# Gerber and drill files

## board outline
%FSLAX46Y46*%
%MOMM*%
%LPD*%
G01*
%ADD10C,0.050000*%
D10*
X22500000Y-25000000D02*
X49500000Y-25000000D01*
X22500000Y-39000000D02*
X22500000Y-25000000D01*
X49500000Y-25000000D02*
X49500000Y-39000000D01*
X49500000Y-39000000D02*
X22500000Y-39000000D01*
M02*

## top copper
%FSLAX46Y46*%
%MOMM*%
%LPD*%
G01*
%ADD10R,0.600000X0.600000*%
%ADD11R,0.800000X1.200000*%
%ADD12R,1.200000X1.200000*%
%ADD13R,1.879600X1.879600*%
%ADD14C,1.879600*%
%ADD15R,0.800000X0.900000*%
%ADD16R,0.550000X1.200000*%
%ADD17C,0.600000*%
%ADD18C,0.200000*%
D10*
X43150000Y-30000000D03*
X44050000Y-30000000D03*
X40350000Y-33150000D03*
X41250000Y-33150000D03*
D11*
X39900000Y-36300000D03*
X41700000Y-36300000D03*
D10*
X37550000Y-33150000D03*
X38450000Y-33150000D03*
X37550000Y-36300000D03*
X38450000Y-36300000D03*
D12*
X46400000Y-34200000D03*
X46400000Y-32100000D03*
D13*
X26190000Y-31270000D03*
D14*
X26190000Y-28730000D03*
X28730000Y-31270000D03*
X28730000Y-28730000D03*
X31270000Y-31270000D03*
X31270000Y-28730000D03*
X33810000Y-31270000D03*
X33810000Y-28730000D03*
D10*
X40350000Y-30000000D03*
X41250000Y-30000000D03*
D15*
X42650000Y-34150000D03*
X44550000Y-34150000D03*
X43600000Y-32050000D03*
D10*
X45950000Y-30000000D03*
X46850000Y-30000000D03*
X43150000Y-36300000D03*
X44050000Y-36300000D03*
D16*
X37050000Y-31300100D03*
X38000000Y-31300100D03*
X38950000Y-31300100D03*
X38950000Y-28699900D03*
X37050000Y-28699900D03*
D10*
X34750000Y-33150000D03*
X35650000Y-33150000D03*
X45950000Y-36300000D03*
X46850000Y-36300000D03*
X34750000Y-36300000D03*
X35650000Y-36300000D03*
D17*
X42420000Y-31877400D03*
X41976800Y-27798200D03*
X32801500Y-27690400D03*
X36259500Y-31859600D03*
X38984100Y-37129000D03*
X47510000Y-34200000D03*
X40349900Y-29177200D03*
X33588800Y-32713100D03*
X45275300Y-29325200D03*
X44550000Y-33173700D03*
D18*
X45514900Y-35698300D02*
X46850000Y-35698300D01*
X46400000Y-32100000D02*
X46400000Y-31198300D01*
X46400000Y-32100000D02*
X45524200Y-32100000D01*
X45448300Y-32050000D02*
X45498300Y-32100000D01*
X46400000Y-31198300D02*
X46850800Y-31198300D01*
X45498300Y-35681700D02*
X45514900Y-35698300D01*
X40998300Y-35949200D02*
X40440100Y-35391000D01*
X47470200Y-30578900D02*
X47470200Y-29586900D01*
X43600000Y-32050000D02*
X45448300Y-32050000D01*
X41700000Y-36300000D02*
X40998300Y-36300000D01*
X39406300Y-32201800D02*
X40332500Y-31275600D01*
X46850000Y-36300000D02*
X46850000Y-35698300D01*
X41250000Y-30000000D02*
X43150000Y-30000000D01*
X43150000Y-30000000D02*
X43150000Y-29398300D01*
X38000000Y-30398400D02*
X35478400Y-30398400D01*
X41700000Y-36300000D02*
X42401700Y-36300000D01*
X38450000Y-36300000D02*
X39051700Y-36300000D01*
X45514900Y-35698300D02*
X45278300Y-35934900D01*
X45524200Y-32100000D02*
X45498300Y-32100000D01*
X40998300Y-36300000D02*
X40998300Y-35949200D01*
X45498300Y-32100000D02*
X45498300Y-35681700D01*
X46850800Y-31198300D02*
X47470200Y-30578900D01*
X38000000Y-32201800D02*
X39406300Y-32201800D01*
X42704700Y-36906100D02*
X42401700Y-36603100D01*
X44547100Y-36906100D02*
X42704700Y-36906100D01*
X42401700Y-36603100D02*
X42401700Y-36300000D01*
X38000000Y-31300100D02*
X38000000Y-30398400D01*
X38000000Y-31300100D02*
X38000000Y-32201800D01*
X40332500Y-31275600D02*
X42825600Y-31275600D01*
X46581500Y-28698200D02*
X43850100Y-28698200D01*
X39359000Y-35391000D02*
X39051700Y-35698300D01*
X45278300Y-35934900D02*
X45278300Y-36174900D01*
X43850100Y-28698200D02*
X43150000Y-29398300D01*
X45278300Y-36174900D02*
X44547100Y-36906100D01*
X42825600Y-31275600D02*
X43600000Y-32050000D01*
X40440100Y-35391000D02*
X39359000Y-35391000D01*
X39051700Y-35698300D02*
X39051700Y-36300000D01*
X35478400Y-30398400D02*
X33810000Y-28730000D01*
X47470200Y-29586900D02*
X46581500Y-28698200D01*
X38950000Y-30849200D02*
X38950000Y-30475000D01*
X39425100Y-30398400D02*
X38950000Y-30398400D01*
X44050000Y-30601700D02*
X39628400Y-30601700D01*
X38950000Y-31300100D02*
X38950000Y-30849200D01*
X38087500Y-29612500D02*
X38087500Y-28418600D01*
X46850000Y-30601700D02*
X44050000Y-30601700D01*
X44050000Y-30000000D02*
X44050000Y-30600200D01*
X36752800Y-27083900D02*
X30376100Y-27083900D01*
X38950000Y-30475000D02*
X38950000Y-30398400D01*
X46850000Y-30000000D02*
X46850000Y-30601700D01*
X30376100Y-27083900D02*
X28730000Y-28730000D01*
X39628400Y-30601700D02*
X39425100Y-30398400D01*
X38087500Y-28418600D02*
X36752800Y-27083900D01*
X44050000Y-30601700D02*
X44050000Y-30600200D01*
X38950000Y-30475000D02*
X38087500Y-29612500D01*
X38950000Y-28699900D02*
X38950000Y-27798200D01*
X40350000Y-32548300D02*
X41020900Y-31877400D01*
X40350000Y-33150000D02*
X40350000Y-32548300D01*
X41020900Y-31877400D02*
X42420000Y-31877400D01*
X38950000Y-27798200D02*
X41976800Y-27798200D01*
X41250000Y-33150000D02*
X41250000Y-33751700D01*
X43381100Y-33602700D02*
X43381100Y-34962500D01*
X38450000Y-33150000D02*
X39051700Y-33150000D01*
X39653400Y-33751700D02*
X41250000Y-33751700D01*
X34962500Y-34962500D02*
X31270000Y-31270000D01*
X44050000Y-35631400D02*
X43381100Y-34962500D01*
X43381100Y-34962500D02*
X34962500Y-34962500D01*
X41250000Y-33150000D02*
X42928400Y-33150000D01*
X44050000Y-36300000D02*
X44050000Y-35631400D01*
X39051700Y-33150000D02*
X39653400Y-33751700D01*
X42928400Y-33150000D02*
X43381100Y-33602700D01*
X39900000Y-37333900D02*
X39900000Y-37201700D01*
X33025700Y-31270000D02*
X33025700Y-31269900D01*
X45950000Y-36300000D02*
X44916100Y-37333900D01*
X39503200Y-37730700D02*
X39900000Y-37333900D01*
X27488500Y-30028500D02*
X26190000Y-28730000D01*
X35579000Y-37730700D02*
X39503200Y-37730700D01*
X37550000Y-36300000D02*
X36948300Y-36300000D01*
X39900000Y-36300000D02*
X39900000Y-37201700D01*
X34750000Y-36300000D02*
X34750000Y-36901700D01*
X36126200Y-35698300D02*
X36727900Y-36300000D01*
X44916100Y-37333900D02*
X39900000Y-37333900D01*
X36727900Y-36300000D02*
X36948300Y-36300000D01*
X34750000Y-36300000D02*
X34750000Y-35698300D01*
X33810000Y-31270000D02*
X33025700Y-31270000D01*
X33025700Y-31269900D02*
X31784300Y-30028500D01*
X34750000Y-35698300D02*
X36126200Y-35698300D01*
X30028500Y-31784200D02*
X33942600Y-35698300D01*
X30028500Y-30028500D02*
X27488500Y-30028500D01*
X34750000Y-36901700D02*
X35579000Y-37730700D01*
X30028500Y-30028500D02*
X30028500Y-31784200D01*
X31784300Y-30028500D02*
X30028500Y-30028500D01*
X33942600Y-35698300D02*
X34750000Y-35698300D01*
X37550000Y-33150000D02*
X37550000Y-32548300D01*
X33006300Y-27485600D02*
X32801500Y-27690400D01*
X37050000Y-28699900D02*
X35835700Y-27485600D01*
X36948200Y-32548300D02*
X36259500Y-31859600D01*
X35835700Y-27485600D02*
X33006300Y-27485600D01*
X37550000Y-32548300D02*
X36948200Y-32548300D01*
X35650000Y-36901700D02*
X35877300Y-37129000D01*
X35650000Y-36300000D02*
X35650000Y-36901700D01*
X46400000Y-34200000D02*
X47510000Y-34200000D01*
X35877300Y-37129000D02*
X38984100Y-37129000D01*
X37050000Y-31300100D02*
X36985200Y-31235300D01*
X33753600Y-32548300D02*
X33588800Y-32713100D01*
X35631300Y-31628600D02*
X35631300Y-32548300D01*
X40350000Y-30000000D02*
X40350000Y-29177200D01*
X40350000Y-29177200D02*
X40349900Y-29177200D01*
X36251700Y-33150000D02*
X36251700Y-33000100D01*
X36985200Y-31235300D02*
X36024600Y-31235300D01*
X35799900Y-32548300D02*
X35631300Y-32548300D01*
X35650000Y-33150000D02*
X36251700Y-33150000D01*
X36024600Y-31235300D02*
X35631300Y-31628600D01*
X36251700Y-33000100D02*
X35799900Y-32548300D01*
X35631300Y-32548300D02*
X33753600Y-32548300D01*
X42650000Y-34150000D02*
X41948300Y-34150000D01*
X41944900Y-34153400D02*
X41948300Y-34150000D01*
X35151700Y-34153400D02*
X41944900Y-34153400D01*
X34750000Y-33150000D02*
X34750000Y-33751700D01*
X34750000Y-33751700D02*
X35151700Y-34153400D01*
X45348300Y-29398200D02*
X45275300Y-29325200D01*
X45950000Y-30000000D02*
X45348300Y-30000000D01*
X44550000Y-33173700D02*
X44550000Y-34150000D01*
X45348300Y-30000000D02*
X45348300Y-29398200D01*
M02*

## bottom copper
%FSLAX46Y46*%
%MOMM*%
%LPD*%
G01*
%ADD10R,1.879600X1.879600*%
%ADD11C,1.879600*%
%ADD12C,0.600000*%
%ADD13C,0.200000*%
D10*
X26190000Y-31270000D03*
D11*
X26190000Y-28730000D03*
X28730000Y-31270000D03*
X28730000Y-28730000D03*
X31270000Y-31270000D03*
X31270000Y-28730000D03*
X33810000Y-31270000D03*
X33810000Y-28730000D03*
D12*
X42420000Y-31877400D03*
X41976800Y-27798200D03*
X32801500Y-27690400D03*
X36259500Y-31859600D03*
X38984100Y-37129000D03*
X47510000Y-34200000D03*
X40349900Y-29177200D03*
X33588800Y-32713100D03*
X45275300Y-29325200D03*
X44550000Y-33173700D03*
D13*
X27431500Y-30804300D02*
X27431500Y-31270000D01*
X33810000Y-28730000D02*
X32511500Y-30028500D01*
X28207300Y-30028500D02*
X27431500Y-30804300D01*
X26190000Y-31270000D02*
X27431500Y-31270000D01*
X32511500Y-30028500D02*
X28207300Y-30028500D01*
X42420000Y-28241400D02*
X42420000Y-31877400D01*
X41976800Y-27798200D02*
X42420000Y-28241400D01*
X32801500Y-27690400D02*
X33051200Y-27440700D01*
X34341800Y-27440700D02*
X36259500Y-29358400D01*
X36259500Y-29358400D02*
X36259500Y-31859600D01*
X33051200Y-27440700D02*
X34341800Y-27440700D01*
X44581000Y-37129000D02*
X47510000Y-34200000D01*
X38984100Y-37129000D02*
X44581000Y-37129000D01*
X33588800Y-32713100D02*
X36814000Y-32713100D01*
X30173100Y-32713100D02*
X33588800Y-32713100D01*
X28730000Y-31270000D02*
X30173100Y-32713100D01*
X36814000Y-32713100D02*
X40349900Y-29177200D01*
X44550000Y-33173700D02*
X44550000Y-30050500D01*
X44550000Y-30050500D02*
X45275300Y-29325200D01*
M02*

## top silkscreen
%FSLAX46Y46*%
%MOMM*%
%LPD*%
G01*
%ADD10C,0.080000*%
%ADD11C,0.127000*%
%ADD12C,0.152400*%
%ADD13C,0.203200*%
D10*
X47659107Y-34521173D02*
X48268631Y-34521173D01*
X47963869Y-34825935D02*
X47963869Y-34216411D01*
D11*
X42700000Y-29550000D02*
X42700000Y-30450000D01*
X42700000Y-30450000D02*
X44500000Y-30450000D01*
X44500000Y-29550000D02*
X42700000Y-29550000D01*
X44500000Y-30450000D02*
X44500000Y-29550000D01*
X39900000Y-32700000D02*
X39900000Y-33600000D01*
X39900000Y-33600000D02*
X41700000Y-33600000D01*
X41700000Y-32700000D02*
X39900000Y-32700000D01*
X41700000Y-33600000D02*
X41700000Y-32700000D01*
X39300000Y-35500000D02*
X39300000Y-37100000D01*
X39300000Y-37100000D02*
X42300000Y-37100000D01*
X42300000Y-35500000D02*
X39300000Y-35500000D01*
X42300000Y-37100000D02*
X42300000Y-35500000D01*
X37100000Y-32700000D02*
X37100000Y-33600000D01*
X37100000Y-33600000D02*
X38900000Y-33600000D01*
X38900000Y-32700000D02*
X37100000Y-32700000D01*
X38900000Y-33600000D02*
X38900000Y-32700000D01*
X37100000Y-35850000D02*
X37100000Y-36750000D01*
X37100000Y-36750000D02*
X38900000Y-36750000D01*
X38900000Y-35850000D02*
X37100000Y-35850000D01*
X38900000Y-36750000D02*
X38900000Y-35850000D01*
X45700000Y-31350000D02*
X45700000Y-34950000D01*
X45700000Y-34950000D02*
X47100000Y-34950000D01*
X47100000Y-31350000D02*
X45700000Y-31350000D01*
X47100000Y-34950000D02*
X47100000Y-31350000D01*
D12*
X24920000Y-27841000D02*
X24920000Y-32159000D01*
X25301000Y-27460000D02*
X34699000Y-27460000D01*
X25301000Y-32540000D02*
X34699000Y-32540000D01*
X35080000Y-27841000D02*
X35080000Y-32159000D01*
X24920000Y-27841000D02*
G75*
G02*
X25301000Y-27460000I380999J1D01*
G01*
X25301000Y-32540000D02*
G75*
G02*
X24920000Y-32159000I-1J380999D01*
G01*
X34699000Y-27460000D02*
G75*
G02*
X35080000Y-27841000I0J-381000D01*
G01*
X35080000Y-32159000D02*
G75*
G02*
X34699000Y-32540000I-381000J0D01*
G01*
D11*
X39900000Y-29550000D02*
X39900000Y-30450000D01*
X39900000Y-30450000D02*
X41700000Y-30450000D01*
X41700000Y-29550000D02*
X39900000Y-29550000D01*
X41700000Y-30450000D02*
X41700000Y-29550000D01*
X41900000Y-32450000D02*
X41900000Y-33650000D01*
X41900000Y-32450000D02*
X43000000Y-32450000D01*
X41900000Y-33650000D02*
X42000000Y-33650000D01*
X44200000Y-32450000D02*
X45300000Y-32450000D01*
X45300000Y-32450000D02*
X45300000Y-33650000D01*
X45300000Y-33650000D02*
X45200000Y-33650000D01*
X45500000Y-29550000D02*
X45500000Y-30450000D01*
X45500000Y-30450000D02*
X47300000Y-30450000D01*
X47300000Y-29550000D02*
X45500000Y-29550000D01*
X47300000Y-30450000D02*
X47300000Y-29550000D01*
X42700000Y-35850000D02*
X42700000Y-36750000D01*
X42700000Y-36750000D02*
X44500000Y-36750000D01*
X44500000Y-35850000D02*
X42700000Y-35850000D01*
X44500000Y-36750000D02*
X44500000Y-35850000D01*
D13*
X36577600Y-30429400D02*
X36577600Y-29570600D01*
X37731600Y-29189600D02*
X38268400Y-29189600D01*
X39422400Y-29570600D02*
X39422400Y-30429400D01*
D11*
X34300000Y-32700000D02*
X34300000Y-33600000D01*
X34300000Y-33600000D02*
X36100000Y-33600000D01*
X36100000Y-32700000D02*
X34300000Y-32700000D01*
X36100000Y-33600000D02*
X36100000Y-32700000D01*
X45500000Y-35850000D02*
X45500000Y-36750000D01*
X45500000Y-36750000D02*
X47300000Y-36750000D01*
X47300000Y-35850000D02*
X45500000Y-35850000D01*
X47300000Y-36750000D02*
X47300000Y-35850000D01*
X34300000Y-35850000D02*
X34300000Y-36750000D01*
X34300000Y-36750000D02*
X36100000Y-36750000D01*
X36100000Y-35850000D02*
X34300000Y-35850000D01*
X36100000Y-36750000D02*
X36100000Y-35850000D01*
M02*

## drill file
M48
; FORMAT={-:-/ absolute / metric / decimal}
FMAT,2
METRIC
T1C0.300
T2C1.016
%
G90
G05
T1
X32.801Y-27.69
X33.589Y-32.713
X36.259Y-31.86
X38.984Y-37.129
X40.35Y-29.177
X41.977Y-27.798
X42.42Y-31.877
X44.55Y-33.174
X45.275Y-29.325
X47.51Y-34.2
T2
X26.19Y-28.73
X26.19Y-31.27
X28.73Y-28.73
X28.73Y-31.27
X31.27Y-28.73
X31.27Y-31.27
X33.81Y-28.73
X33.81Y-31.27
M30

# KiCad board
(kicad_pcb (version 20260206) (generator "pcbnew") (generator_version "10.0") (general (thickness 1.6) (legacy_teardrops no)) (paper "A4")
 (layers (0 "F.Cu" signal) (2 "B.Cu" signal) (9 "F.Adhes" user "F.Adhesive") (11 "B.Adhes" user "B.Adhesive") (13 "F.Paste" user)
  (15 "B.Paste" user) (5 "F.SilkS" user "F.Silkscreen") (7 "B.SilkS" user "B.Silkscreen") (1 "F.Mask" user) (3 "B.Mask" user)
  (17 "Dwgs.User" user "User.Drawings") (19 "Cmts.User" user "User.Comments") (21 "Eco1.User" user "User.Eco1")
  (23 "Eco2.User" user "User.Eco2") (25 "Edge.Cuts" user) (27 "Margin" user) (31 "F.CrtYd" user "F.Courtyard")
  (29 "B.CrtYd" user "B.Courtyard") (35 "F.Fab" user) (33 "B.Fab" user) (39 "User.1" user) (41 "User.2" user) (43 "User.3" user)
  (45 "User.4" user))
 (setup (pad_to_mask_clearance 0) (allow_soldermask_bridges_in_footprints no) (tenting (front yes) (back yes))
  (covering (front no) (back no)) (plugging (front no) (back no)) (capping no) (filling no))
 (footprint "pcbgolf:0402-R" (layer "F.Cu") (at 43.6 30)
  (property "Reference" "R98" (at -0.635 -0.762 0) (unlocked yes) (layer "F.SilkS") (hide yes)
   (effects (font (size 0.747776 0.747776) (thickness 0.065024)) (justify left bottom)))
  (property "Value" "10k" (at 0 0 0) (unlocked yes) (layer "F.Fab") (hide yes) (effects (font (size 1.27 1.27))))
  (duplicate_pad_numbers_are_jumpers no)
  (fp_line (start -0.9 -0.45) (end -0.9 0.45) (stroke (width 0.127) (type solid)) (layer "F.SilkS"))
  (fp_line (start -0.9 0.45) (end 0.9 0.45) (stroke (width 0.127) (type solid)) (layer "F.SilkS"))
  (fp_line (start 0.9 -0.45) (end -0.9 -0.45) (stroke (width 0.127) (type solid)) (layer "F.SilkS"))
  (fp_line (start 0.9 0.45) (end 0.9 -0.45) (stroke (width 0.127) (type solid)) (layer "F.SilkS"))
  (pad "1" smd rect (at -0.45 0) (size 0.6 0.6) (layers "F.Cu" "F.Mask" "F.Paste") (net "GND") (solder_mask_margin 0.0508)
   (solder_paste_margin 0) (thermal_bridge_angle 0))
  (pad "2" smd rect (at 0.45 0) (size 0.6 0.6) (layers "F.Cu" "F.Mask" "F.Paste") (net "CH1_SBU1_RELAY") (solder_mask_margin 0.0508)
   (solder_paste_margin 0) (thermal_bridge_angle 0)))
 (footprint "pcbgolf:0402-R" (layer "F.Cu") (at 40.8 33.15)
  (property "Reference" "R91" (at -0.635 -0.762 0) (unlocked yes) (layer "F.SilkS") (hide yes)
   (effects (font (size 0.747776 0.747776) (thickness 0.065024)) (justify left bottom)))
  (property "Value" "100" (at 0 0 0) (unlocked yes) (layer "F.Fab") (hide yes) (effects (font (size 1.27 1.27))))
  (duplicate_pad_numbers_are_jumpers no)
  (fp_line (start -0.9 -0.45) (end -0.9 0.45) (stroke (width 0.127) (type solid)) (layer "F.SilkS"))
  (fp_line (start -0.9 0.45) (end 0.9 0.45) (stroke (width 0.127) (type solid)) (layer "F.SilkS"))
  (fp_line (start 0.9 -0.45) (end -0.9 -0.45) (stroke (width 0.127) (type solid)) (layer "F.SilkS"))
  (fp_line (start 0.9 0.45) (end 0.9 -0.45) (stroke (width 0.127) (type solid)) (layer "F.SilkS"))
  (pad "1" smd rect (at -0.45 0) (size 0.6 0.6) (layers "F.Cu" "F.Mask" "F.Paste") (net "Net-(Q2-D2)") (solder_mask_margin 0.0508)
   (solder_paste_margin 0) (thermal_bridge_angle 0))
  (pad "2" smd rect (at 0.45 0) (size 0.6 0.6) (layers "F.Cu" "F.Mask" "F.Paste") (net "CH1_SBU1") (solder_mask_margin 0.0508)
   (solder_paste_margin 0) (thermal_bridge_angle 0)))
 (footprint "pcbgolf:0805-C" (layer "F.Cu") (at 40.8 36.3)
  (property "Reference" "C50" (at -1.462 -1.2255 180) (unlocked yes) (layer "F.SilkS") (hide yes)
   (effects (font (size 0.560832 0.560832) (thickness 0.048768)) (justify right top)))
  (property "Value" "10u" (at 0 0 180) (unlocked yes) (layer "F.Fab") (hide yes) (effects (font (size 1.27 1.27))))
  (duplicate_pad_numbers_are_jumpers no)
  (fp_line (start -1.5 -0.8) (end -1.5 0.8) (stroke (width 0.127) (type solid)) (layer "F.SilkS"))
  (fp_line (start -1.5 0.8) (end 1.5 0.8) (stroke (width 0.127) (type solid)) (layer "F.SilkS"))
  (fp_line (start 1.5 -0.8) (end -1.5 -0.8) (stroke (width 0.127) (type solid)) (layer "F.SilkS"))
  (fp_line (start 1.5 0.8) (end 1.5 -0.8) (stroke (width 0.127) (type solid)) (layer "F.SilkS"))
  (pad "1" smd rect (at -0.9 0) (size 0.8 1.2) (layers "F.Cu" "F.Mask" "F.Paste") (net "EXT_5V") (solder_mask_margin 0.0508)
   (solder_paste_margin 0) (thermal_bridge_angle 0))
  (pad "2" smd rect (at 0.9 0) (size 0.8 1.2) (layers "F.Cu" "F.Mask" "F.Paste") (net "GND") (solder_mask_margin 0.0508)
   (solder_paste_margin 0) (thermal_bridge_angle 0)))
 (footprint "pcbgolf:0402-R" (layer "F.Cu") (at 38 33.15)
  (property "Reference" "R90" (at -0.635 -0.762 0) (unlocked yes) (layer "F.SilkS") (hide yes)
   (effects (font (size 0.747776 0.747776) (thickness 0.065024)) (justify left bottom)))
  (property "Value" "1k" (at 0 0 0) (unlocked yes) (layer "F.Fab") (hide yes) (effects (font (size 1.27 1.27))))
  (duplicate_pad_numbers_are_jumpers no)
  (fp_line (start -0.9 -0.45) (end -0.9 0.45) (stroke (width 0.127) (type solid)) (layer "F.SilkS"))
  (fp_line (start -0.9 0.45) (end 0.9 0.45) (stroke (width 0.127) (type solid)) (layer "F.SilkS"))
  (fp_line (start 0.9 -0.45) (end -0.9 -0.45) (stroke (width 0.127) (type solid)) (layer "F.SilkS"))
  (fp_line (start 0.9 0.45) (end 0.9 -0.45) (stroke (width 0.127) (type solid)) (layer "F.SilkS"))
  (pad "1" smd rect (at -0.45 0) (size 0.6 0.6) (layers "F.Cu" "F.Mask" "F.Paste") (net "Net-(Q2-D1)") (solder_mask_margin 0.0508)
   (solder_paste_margin 0) (thermal_bridge_angle 0))
  (pad "2" smd rect (at 0.45 0) (size 0.6 0.6) (layers "F.Cu" "F.Mask" "F.Paste") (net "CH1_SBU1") (solder_mask_margin 0.0508)
   (solder_paste_margin 0) (thermal_bridge_angle 0)))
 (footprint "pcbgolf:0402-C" (layer "F.Cu") (at 38 36.3)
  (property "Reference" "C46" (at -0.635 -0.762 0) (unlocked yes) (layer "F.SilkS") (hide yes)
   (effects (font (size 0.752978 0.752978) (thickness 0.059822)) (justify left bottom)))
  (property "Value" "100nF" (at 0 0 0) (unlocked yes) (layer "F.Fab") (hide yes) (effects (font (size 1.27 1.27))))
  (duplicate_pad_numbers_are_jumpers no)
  (fp_line (start -0.9 -0.45) (end -0.9 0.45) (stroke (width 0.127) (type solid)) (layer "F.SilkS"))
  (fp_line (start -0.9 0.45) (end 0.9 0.45) (stroke (width 0.127) (type solid)) (layer "F.SilkS"))
  (fp_line (start 0.9 -0.45) (end -0.9 -0.45) (stroke (width 0.127) (type solid)) (layer "F.SilkS"))
  (fp_line (start 0.9 0.45) (end 0.9 -0.45) (stroke (width 0.127) (type solid)) (layer "F.SilkS"))
  (pad "1" smd rect (at -0.45 0) (size 0.6 0.6) (layers "F.Cu" "F.Mask" "F.Paste") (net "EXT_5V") (solder_mask_margin 0.0508)
   (solder_paste_margin 0) (thermal_bridge_angle 0))
  (pad "2" smd rect (at 0.45 0) (size 0.6 0.6) (layers "F.Cu" "F.Mask" "F.Paste") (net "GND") (solder_mask_margin 0.0508)
   (solder_paste_margin 0) (thermal_bridge_angle 0)))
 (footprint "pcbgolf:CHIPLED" (layer "F.Cu") (at 46.4 33.15)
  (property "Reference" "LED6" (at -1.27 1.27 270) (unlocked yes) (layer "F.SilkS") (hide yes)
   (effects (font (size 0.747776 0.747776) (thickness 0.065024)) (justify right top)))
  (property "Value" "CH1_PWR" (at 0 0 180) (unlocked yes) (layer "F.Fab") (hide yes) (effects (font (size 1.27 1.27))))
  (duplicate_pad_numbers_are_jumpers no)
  (fp_line (start -0.7 -1.8) (end -0.7 1.8) (stroke (width 0.127) (type solid)) (layer "F.SilkS"))
  (fp_line (start -0.7 1.8) (end 0.7 1.8) (stroke (width 0.127) (type solid)) (layer "F.SilkS"))
  (fp_line (start 0.7 -1.8) (end -0.7 -1.8) (stroke (width 0.127) (type solid)) (layer "F.SilkS"))
  (fp_line (start 0.7 1.8) (end 0.7 -1.8) (stroke (width 0.127) (type solid)) (layer "F.SilkS"))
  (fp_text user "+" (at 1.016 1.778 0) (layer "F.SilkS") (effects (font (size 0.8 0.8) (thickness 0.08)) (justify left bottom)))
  (pad "A" smd rect (at 0 1.05) (size 1.2 1.2) (layers "F.Cu" "F.Mask" "F.Paste") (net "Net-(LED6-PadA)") (solder_mask_margin 0.0508)
   (solder_paste_margin 0) (thermal_bridge_angle 0))
  (pad "C" smd rect (at 0 -1.05) (size 1.2 1.2) (layers "F.Cu" "F.Mask" "F.Paste") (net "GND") (solder_mask_margin 0.0508)
   (solder_paste_margin 0) (thermal_bridge_angle 0)))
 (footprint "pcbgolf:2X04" (layer "F.Cu") (at 30 30)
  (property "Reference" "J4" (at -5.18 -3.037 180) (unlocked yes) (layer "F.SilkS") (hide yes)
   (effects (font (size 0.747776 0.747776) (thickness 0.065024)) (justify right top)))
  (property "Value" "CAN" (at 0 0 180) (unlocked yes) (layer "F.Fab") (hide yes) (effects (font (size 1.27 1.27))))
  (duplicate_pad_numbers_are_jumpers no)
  (fp_line (start -5.08 -2.159) (end -5.08 2.159) (stroke (width 0.1524) (type solid)) (layer "F.SilkS"))
  (fp_line (start -4.699 -2.54) (end 4.699 -2.54) (stroke (width 0.1524) (type solid)) (layer "F.SilkS"))
  (fp_line (start -4.699 2.54) (end 4.699 2.54) (stroke (width 0.1524) (type solid)) (layer "F.SilkS"))
  (fp_line (start 5.08 -2.159) (end 5.08 2.159) (stroke (width 0.1524) (type solid)) (layer "F.SilkS"))
  (fp_arc (start -5.08 -2.159) (mid -4.968408 -2.428408) (end -4.699 -2.54) (stroke (width 0.1524) (type solid)) (layer "F.SilkS"))
  (fp_arc (start -4.699 2.54) (mid -4.968408 2.428408) (end -5.08 2.159) (stroke (width 0.1524) (type solid)) (layer "F.SilkS"))
  (fp_arc (start 4.699 -2.54) (mid 4.968408 -2.428408) (end 5.08 -2.159) (stroke (width 0.1524) (type solid)) (layer "F.SilkS"))
  (fp_arc (start 5.08 2.159) (mid 4.968408 2.428408) (end 4.699 2.54) (stroke (width 0.1524) (type solid)) (layer "F.SilkS"))
  (pad "1" thru_hole rect (at -3.81 1.27 90) (size 1.8796 1.8796) (drill 1.016) (layers "*.Cu" "*.Mask") (remove_unused_layers no)
   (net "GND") (solder_mask_margin 0.0508) (thermal_bridge_angle 0))
  (pad "2" thru_hole circle (at -3.81 -1.27 90) (size 1.8796 1.8796) (drill 1.016) (layers "*.Cu" "*.Mask") (remove_unused_layers no)
   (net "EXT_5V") (solder_mask_margin 0.0508) (thermal_bridge_angle 0))
  (pad "3" thru_hole circle (at -1.27 1.27 90) (size 1.8796 1.8796) (drill 1.016) (layers "*.Cu" "*.Mask") (remove_unused_layers no)
   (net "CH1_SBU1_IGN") (solder_mask_margin 0.0508) (thermal_bridge_angle 0))
  (pad "4" thru_hole circle (at -1.27 -1.27 90) (size 1.8796 1.8796) (drill 1.016) (layers "*.Cu" "*.Mask") (remove_unused_layers no)
   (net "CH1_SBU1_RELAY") (solder_mask_margin 0.0508) (thermal_bridge_angle 0))
  (pad "5" thru_hole circle (at 1.27 1.27 90) (size 1.8796 1.8796) (drill 1.016) (layers "*.Cu" "*.Mask") (remove_unused_layers no)
   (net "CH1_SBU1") (solder_mask_margin 0.0508) (thermal_bridge_angle 0))
  (pad "6" thru_hole circle (at 1.27 -1.27 90) (size 1.8796 1.8796) (drill 1.016) (layers "*.Cu" "*.Mask") (remove_unused_layers no)
   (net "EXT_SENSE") (solder_mask_margin 0.0508) (thermal_bridge_angle 0))
  (pad "7" thru_hole circle (at 3.81 1.27 90) (size 1.8796 1.8796) (drill 1.016) (layers "*.Cu" "*.Mask") (remove_unused_layers no)
   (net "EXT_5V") (solder_mask_margin 0.0508) (thermal_bridge_angle 0))
  (pad "8" thru_hole circle (at 3.81 -1.27 90) (size 1.8796 1.8796) (drill 1.016) (layers "*.Cu" "*.Mask") (remove_unused_layers no)
   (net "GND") (solder_mask_margin 0.0508) (thermal_bridge_angle 0)))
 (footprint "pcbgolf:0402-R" (layer "F.Cu") (at 40.8 30)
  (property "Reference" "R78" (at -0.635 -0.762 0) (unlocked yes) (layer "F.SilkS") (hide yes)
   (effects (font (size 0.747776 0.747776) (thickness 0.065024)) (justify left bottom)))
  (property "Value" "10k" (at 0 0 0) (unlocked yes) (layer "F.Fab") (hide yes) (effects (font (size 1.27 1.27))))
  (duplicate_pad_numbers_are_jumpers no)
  (fp_line (start -0.9 -0.45) (end -0.9 0.45) (stroke (width 0.127) (type solid)) (layer "F.SilkS"))
  (fp_line (start -0.9 0.45) (end 0.9 0.45) (stroke (width 0.127) (type solid)) (layer "F.SilkS"))
  (fp_line (start 0.9 -0.45) (end -0.9 -0.45) (stroke (width 0.127) (type solid)) (layer "F.SilkS"))
  (fp_line (start 0.9 0.45) (end 0.9 -0.45) (stroke (width 0.127) (type solid)) (layer "F.SilkS"))
  (pad "1" smd rect (at -0.45 0) (size 0.6 0.6) (layers "F.Cu" "F.Mask" "F.Paste") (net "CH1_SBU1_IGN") (solder_mask_margin 0.0508)
   (solder_paste_margin 0) (thermal_bridge_angle 0))
  (pad "2" smd rect (at 0.45 0) (size 0.6 0.6) (layers "F.Cu" "F.Mask" "F.Paste") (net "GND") (solder_mask_margin 0.0508)
   (solder_paste_margin 0) (thermal_bridge_angle 0)))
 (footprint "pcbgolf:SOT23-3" (layer "F.Cu") (at 43.6 33.15)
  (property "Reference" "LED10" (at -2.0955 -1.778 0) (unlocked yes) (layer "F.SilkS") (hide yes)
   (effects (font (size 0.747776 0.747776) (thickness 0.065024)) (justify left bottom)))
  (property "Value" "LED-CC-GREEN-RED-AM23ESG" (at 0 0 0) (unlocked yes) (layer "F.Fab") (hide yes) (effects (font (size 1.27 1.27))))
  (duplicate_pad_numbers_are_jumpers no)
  (fp_line (start -1.7 -0.7) (end -1.7 0.5) (stroke (width 0.127) (type solid)) (layer "F.SilkS"))
  (fp_line (start -1.7 -0.7) (end -0.6 -0.7) (stroke (width 0.127) (type solid)) (layer "F.SilkS"))
  (fp_line (start -1.7 0.5) (end -1.6 0.5) (stroke (width 0.127) (type solid)) (layer "F.SilkS"))
  (fp_line (start 0.6 -0.7) (end 1.7 -0.7) (stroke (width 0.127) (type solid)) (layer "F.SilkS"))
  (fp_line (start 1.7 -0.7) (end 1.7 0.5) (stroke (width 0.127) (type solid)) (layer "F.SilkS"))
  (fp_line (start 1.7 0.5) (end 1.6 0.5) (stroke (width 0.127) (type solid)) (layer "F.SilkS"))
  (pad "1" smd rect (at -0.95 1) (size 0.8 0.9) (layers "F.Cu" "F.Mask" "F.Paste") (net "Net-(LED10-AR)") (solder_mask_margin 0.0508)
   (solder_paste_margin 0) (thermal_bridge_angle 0))
  (pad "2" smd rect (at 0.95 1) (size 0.8 0.9) (layers "F.Cu" "F.Mask" "F.Paste") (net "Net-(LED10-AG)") (solder_mask_margin 0.0508)
   (solder_paste_margin 0) (thermal_bridge_angle 0))
  (pad "3" smd rect (at 0 -1.1) (size 0.8 0.9) (layers "F.Cu" "F.Mask" "F.Paste") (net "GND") (solder_mask_margin 0.0508)
   (solder_paste_margin 0) (thermal_bridge_angle 0)))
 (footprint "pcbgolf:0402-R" (layer "F.Cu") (at 46.4 30)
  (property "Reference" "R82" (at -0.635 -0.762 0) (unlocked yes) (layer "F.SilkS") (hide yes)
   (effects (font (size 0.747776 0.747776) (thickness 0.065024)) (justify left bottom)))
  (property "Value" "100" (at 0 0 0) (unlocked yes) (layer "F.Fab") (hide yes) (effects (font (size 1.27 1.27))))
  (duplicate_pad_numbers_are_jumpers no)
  (fp_line (start -0.9 -0.45) (end -0.9 0.45) (stroke (width 0.127) (type solid)) (layer "F.SilkS"))
  (fp_line (start -0.9 0.45) (end 0.9 0.45) (stroke (width 0.127) (type solid)) (layer "F.SilkS"))
  (fp_line (start 0.9 -0.45) (end -0.9 -0.45) (stroke (width 0.127) (type solid)) (layer "F.SilkS"))
  (fp_line (start 0.9 0.45) (end 0.9 -0.45) (stroke (width 0.127) (type solid)) (layer "F.SilkS"))
  (pad "1" smd rect (at -0.45 0) (size 0.6 0.6) (layers "F.Cu" "F.Mask" "F.Paste") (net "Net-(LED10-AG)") (solder_mask_margin 0.0508)
   (solder_paste_margin 0) (thermal_bridge_angle 0))
  (pad "2" smd rect (at 0.45 0) (size 0.6 0.6) (layers "F.Cu" "F.Mask" "F.Paste") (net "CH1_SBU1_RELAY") (solder_mask_margin 0.0508)
   (solder_paste_margin 0) (thermal_bridge_angle 0)))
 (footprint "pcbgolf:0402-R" (layer "F.Cu") (at 43.6 36.3)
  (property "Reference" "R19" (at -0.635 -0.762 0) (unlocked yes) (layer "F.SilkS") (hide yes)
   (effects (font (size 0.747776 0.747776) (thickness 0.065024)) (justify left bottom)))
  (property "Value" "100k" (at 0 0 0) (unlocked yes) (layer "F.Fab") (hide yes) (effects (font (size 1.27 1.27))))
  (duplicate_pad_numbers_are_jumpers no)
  (fp_line (start -0.9 -0.45) (end -0.9 0.45) (stroke (width 0.127) (type solid)) (layer "F.SilkS"))
  (fp_line (start -0.9 0.45) (end 0.9 0.45) (stroke (width 0.127) (type solid)) (layer "F.SilkS"))
  (fp_line (start 0.9 -0.45) (end -0.9 -0.45) (stroke (width 0.127) (type solid)) (layer "F.SilkS"))
  (fp_line (start 0.9 0.45) (end 0.9 -0.45) (stroke (width 0.127) (type solid)) (layer "F.SilkS"))
  (pad "1" smd rect (at -0.45 0) (size 0.6 0.6) (layers "F.Cu" "F.Mask" "F.Paste") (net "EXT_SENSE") (solder_mask_margin 0.0508)
   (solder_paste_margin 0) (thermal_bridge_angle 0))
  (pad "2" smd rect (at 0.45 0) (size 0.6 0.6) (layers "F.Cu" "F.Mask" "F.Paste") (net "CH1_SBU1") (solder_mask_margin 0.0508)
   (solder_paste_margin 0) (thermal_bridge_angle 0)))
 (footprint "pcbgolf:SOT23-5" (layer "F.Cu") (at 38 30)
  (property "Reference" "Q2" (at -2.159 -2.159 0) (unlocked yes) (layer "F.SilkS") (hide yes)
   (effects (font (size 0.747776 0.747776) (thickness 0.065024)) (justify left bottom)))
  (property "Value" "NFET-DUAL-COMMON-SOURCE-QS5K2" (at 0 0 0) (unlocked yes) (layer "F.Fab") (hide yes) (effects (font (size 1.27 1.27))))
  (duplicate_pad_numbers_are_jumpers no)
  (fp_line (start -1.4224 0.4294) (end -1.4224 -0.4294) (stroke (width 0.2032) (type solid)) (layer "F.SilkS"))
  (fp_line (start -0.2684 -0.8104) (end 0.2684 -0.8104) (stroke (width 0.2032) (type solid)) (layer "F.SilkS"))
  (fp_line (start 1.4224 -0.4294) (end 1.4224 0.4294) (stroke (width 0.2032) (type solid)) (layer "F.SilkS"))
  (pad "1" smd rect (at -0.95 1.3001) (size 0.55 1.2) (layers "F.Cu" "F.Mask" "F.Paste") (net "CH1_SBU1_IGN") (solder_mask_margin 0.0508)
   (solder_paste_margin 0) (thermal_bridge_angle 0))
  (pad "2" smd rect (at 0 1.3001) (size 0.55 1.2) (layers "F.Cu" "F.Mask" "F.Paste") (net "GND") (solder_mask_margin 0.0508)
   (solder_paste_margin 0) (thermal_bridge_angle 0))
  (pad "3" smd rect (at 0.95 1.3001) (size 0.55 1.2) (layers "F.Cu" "F.Mask" "F.Paste") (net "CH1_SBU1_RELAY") (solder_mask_margin 0.0508)
   (solder_paste_margin 0) (thermal_bridge_angle 0))
  (pad "4" smd rect (at 0.95 -1.3001) (size 0.55 1.2) (layers "F.Cu" "F.Mask" "F.Paste") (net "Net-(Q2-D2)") (solder_mask_margin 0.0508)
   (solder_paste_margin 0) (thermal_bridge_angle 0))
  (pad "5" smd rect (at -0.95 -1.3001) (size 0.55 1.2) (layers "F.Cu" "F.Mask" "F.Paste") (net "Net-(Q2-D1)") (solder_mask_margin 0.0508)
   (solder_paste_margin 0) (thermal_bridge_angle 0)))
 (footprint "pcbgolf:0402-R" (layer "F.Cu") (at 35.2 33.15)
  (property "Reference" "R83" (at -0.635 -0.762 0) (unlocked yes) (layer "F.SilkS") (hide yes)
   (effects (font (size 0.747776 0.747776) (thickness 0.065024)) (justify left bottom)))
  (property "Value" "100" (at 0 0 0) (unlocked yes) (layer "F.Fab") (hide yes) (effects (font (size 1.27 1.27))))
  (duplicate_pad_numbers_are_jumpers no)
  (fp_line (start -0.9 -0.45) (end -0.9 0.45) (stroke (width 0.127) (type solid)) (layer "F.SilkS"))
  (fp_line (start -0.9 0.45) (end 0.9 0.45) (stroke (width 0.127) (type solid)) (layer "F.SilkS"))
  (fp_line (start 0.9 -0.45) (end -0.9 -0.45) (stroke (width 0.127) (type solid)) (layer "F.SilkS"))
  (fp_line (start 0.9 0.45) (end 0.9 -0.45) (stroke (width 0.127) (type solid)) (layer "F.SilkS"))
  (pad "1" smd rect (at -0.45 0) (size 0.6 0.6) (layers "F.Cu" "F.Mask" "F.Paste") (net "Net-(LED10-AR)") (solder_mask_margin 0.0508)
   (solder_paste_margin 0) (thermal_bridge_angle 0))
  (pad "2" smd rect (at 0.45 0) (size 0.6 0.6) (layers "F.Cu" "F.Mask" "F.Paste") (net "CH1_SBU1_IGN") (solder_mask_margin 0.0508)
   (solder_paste_margin 0) (thermal_bridge_angle 0)))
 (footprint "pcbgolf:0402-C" (layer "F.Cu") (at 46.4 36.3)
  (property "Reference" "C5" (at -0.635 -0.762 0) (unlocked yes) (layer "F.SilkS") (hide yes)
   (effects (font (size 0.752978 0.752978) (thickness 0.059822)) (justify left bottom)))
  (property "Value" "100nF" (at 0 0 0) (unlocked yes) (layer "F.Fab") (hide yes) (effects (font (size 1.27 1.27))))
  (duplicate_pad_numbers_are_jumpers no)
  (fp_line (start -0.9 -0.45) (end -0.9 0.45) (stroke (width 0.127) (type solid)) (layer "F.SilkS"))
  (fp_line (start -0.9 0.45) (end 0.9 0.45) (stroke (width 0.127) (type solid)) (layer "F.SilkS"))
  (fp_line (start 0.9 -0.45) (end -0.9 -0.45) (stroke (width 0.127) (type solid)) (layer "F.SilkS"))
  (fp_line (start 0.9 0.45) (end 0.9 -0.45) (stroke (width 0.127) (type solid)) (layer "F.SilkS"))
  (pad "1" smd rect (at -0.45 0) (size 0.6 0.6) (layers "F.Cu" "F.Mask" "F.Paste") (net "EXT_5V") (solder_mask_margin 0.0508)
   (solder_paste_margin 0) (thermal_bridge_angle 0))
  (pad "2" smd rect (at 0.45 0) (size 0.6 0.6) (layers "F.Cu" "F.Mask" "F.Paste") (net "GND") (solder_mask_margin 0.0508)
   (solder_paste_margin 0) (thermal_bridge_angle 0)))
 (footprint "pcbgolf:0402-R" (layer "F.Cu") (at 35.2 36.3)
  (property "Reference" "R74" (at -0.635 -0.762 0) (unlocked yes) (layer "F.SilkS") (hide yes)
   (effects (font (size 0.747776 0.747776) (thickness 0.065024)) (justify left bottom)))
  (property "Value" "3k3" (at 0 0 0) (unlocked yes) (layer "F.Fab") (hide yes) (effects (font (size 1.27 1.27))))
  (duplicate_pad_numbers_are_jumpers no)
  (fp_line (start -0.9 -0.45) (end -0.9 0.45) (stroke (width 0.127) (type solid)) (layer "F.SilkS"))
  (fp_line (start -0.9 0.45) (end 0.9 0.45) (stroke (width 0.127) (type solid)) (layer "F.SilkS"))
  (fp_line (start 0.9 -0.45) (end -0.9 -0.45) (stroke (width 0.127) (type solid)) (layer "F.SilkS"))
  (fp_line (start 0.9 0.45) (end 0.9 -0.45) (stroke (width 0.127) (type solid)) (layer "F.SilkS"))
  (pad "1" smd rect (at -0.45 0) (size 0.6 0.6) (layers "F.Cu" "F.Mask" "F.Paste") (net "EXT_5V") (solder_mask_margin 0.0508)
   (solder_paste_margin 0) (thermal_bridge_angle 0))
  (pad "2" smd rect (at 0.45 0) (size 0.6 0.6) (layers "F.Cu" "F.Mask" "F.Paste") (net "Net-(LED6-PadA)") (solder_mask_margin 0.0508)
   (solder_paste_margin 0) (thermal_bridge_angle 0)))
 (gr_line (start 22.5 25) (end 49.5 25) (stroke (width 0.05) (type default)) (layer "Edge.Cuts"))
 (gr_line (start 22.5 39) (end 22.5 25) (stroke (width 0.05) (type default)) (layer "Edge.Cuts"))
 (gr_line (start 49.5 25) (end 49.5 39) (stroke (width 0.05) (type default)) (layer "Edge.Cuts"))
 (gr_line (start 49.5 39) (end 22.5 39) (stroke (width 0.05) (type default)) (layer "Edge.Cuts"))
 (segment (start 45.5149 35.6983) (end 46.85 35.6983) (width 0.2) (layer "F.Cu") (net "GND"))
 (segment (start 46.4 32.1) (end 46.4 31.1983) (width 0.2) (layer "F.Cu") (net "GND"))
 (segment (start 46.4 32.1) (end 45.5242 32.1) (width 0.2) (layer "F.Cu") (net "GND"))
 (segment (start 45.4483 32.05) (end 45.4983 32.1) (width 0.2) (layer "F.Cu") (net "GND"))
 (segment (start 46.4 31.1983) (end 46.8508 31.1983) (width 0.2) (layer "F.Cu") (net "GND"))
 (segment (start 45.4983 35.6817) (end 45.5149 35.6983) (width 0.2) (layer "F.Cu") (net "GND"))
 (segment (start 40.9983 35.9492) (end 40.4401 35.391) (width 0.2) (layer "F.Cu") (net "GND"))
 (segment (start 47.4702 30.5789) (end 47.4702 29.5869) (width 0.2) (layer "F.Cu") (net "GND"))
 (segment (start 43.6 32.05) (end 45.4483 32.05) (width 0.2) (layer "F.Cu") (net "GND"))
 (segment (start 41.7 36.3) (end 40.9983 36.3) (width 0.2) (layer "F.Cu") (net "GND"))
 (segment (start 39.4063 32.2018) (end 40.3325 31.2756) (width 0.2) (layer "F.Cu") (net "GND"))
 (segment (start 46.85 36.3) (end 46.85 35.6983) (width 0.2) (layer "F.Cu") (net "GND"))
 (segment (start 41.25 30) (end 43.15 30) (width 0.2) (layer "F.Cu") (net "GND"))
 (segment (start 43.15 30) (end 43.15 29.3983) (width 0.2) (layer "F.Cu") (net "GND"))
 (segment (start 38 30.3984) (end 35.4784 30.3984) (width 0.2) (layer "F.Cu") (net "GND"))
 (segment (start 41.7 36.3) (end 42.4017 36.3) (width 0.2) (layer "F.Cu") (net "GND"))
 (segment (start 38.45 36.3) (end 39.0517 36.3) (width 0.2) (layer "F.Cu") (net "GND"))
 (segment (start 45.5149 35.6983) (end 45.2783 35.9349) (width 0.2) (layer "F.Cu") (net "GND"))
 (segment (start 45.5242 32.1) (end 45.4983 32.1) (width 0.2) (layer "F.Cu") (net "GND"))
 (segment (start 40.9983 36.3) (end 40.9983 35.9492) (width 0.2) (layer "F.Cu") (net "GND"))
 (segment (start 45.4983 32.1) (end 45.4983 35.6817) (width 0.2) (layer "F.Cu") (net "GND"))
 (segment (start 46.8508 31.1983) (end 47.4702 30.5789) (width 0.2) (layer "F.Cu") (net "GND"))
 (segment (start 38 32.2018) (end 39.4063 32.2018) (width 0.2) (layer "F.Cu") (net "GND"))
 (segment (start 42.7047 36.9061) (end 42.4017 36.6031) (width 0.2) (layer "F.Cu") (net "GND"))
 (segment (start 44.5471 36.9061) (end 42.7047 36.9061) (width 0.2) (layer "F.Cu") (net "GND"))
 (segment (start 42.4017 36.6031) (end 42.4017 36.3) (width 0.2) (layer "F.Cu") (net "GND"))
 (segment (start 38 31.3001) (end 38 30.3984) (width 0.2) (layer "F.Cu") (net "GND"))
 (segment (start 38 31.3001) (end 38 32.2018) (width 0.2) (layer "F.Cu") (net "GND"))
 (segment (start 40.3325 31.2756) (end 42.8256 31.2756) (width 0.2) (layer "F.Cu") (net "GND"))
 (segment (start 46.5815 28.6982) (end 43.8501 28.6982) (width 0.2) (layer "F.Cu") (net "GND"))
 (segment (start 39.359 35.391) (end 39.0517 35.6983) (width 0.2) (layer "F.Cu") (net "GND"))
 (segment (start 45.2783 35.9349) (end 45.2783 36.1749) (width 0.2) (layer "F.Cu") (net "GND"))
 (segment (start 43.8501 28.6982) (end 43.15 29.3983) (width 0.2) (layer "F.Cu") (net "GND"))
 (segment (start 45.2783 36.1749) (end 44.5471 36.9061) (width 0.2) (layer "F.Cu") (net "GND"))
 (segment (start 42.8256 31.2756) (end 43.6 32.05) (width 0.2) (layer "F.Cu") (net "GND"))
 (segment (start 40.4401 35.391) (end 39.359 35.391) (width 0.2) (layer "F.Cu") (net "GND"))
 (segment (start 39.0517 35.6983) (end 39.0517 36.3) (width 0.2) (layer "F.Cu") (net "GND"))
 (segment (start 35.4784 30.3984) (end 33.81 28.73) (width 0.2) (layer "F.Cu") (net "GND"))
 (segment (start 47.4702 29.5869) (end 46.5815 28.6982) (width 0.2) (layer "F.Cu") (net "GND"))
 (segment (start 27.4315 30.8043) (end 27.4315 31.27) (width 0.2) (layer "B.Cu") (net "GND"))
 (segment (start 33.81 28.73) (end 32.5115 30.0285) (width 0.2) (layer "B.Cu") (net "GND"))
 (segment (start 28.2073 30.0285) (end 27.4315 30.8043) (width 0.2) (layer "B.Cu") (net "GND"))
 (segment (start 26.19 31.27) (end 27.4315 31.27) (width 0.2) (layer "B.Cu") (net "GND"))
 (segment (start 32.5115 30.0285) (end 28.2073 30.0285) (width 0.2) (layer "B.Cu") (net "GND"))
 (segment (start 38.95 30.8492) (end 38.95 30.475) (width 0.2) (layer "F.Cu") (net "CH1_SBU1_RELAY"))
 (segment (start 39.4251 30.3984) (end 38.95 30.3984) (width 0.2) (layer "F.Cu") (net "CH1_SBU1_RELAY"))
 (segment (start 44.05 30.6017) (end 39.6284 30.6017) (width 0.2) (layer "F.Cu") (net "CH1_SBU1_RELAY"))
 (segment (start 38.95 31.3001) (end 38.95 30.8492) (width 0.2) (layer "F.Cu") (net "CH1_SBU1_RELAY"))
 (segment (start 38.0875 29.6125) (end 38.0875 28.4186) (width 0.2) (layer "F.Cu") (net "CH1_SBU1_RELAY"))
 (segment (start 46.85 30.6017) (end 44.05 30.6017) (width 0.2) (layer "F.Cu") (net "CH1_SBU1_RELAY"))
 (segment (start 44.05 30) (end 44.05 30.6002) (width 0.2) (layer "F.Cu") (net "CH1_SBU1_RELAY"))
 (segment (start 36.7528 27.0839) (end 30.3761 27.0839) (width 0.2) (layer "F.Cu") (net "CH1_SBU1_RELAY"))
 (segment (start 38.95 30.475) (end 38.95 30.3984) (width 0.2) (layer "F.Cu") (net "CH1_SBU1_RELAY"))
 (segment (start 46.85 30) (end 46.85 30.6017) (width 0.2) (layer "F.Cu") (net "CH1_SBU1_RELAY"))
 (segment (start 30.3761 27.0839) (end 28.73 28.73) (width 0.2) (layer "F.Cu") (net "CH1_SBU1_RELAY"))
 (segment (start 39.6284 30.6017) (end 39.4251 30.3984) (width 0.2) (layer "F.Cu") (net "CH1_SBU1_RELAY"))
 (segment (start 38.0875 28.4186) (end 36.7528 27.0839) (width 0.2) (layer "F.Cu") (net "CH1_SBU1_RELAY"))
 (segment (start 44.05 30.6017) (end 44.05 30.6002) (width 0.2) (layer "F.Cu") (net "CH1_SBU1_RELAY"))
 (segment (start 38.95 30.475) (end 38.0875 29.6125) (width 0.2) (layer "F.Cu") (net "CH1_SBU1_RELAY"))
 (segment (start 38.95 28.6999) (end 38.95 27.7982) (width 0.2) (layer "F.Cu") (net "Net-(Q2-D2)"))
 (segment (start 40.35 32.5483) (end 41.0209 31.8774) (width 0.2) (layer "F.Cu") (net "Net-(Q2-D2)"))
 (segment (start 40.35 33.15) (end 40.35 32.5483) (width 0.2) (layer "F.Cu") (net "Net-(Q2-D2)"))
 (segment (start 41.0209 31.8774) (end 42.42 31.8774) (width 0.2) (layer "F.Cu") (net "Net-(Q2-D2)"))
 (segment (start 38.95 27.7982) (end 41.9768 27.7982) (width 0.2) (layer "F.Cu") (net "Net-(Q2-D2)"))
 (via (at 42.42 31.8774) (size 0.6) (drill 0.3) (layers "F.Cu" "B.Cu") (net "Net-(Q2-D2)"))
 (via (at 41.9768 27.7982) (size 0.6) (drill 0.3) (layers "F.Cu" "B.Cu") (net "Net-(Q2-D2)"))
 (segment (start 42.42 28.2414) (end 42.42 31.8774) (width 0.2) (layer "B.Cu") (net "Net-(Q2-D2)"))
 (segment (start 41.9768 27.7982) (end 42.42 28.2414) (width 0.2) (layer "B.Cu") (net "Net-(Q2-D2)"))
 (segment (start 41.25 33.15) (end 41.25 33.7517) (width 0.2) (layer "F.Cu") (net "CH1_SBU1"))
 (segment (start 43.3811 33.6027) (end 43.3811 34.9625) (width 0.2) (layer "F.Cu") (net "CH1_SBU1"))
 (segment (start 38.45 33.15) (end 39.0517 33.15) (width 0.2) (layer "F.Cu") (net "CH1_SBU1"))
 (segment (start 39.6534 33.7517) (end 41.25 33.7517) (width 0.2) (layer "F.Cu") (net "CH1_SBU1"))
 (segment (start 34.9625 34.9625) (end 31.27 31.27) (width 0.2) (layer "F.Cu") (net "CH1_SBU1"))
 (segment (start 44.05 35.6314) (end 43.3811 34.9625) (width 0.2) (layer "F.Cu") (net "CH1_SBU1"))
 (segment (start 43.3811 34.9625) (end 34.9625 34.9625) (width 0.2) (layer "F.Cu") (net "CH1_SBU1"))
 (segment (start 41.25 33.15) (end 42.9284 33.15) (width 0.2) (layer "F.Cu") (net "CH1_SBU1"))
 (segment (start 44.05 36.3) (end 44.05 35.6314) (width 0.2) (layer "F.Cu") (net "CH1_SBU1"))
 (segment (start 39.0517 33.15) (end 39.6534 33.7517) (width 0.2) (layer "F.Cu") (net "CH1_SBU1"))
 (segment (start 42.9284 33.15) (end 43.3811 33.6027) (width 0.2) (layer "F.Cu") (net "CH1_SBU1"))
 (segment (start 39.9 37.3339) (end 39.9 37.2017) (width 0.2) (layer "F.Cu") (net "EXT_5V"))
 (segment (start 33.0257 31.27) (end 33.0257 31.2699) (width 0.2) (layer "F.Cu") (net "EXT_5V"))
 (segment (start 45.95 36.3) (end 44.9161 37.3339) (width 0.2) (layer "F.Cu") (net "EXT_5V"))
 (segment (start 39.5032 37.7307) (end 39.9 37.3339) (width 0.2) (layer "F.Cu") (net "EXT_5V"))
 (segment (start 27.4885 30.0285) (end 26.19 28.73) (width 0.2) (layer "F.Cu") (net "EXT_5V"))
 (segment (start 35.579 37.7307) (end 39.5032 37.7307) (width 0.2) (layer "F.Cu") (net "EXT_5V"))
 (segment (start 37.55 36.3) (end 36.9483 36.3) (width 0.2) (layer "F.Cu") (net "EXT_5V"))
 (segment (start 39.9 36.3) (end 39.9 37.2017) (width 0.2) (layer "F.Cu") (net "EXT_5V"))
 (segment (start 34.75 36.3) (end 34.75 36.9017) (width 0.2) (layer "F.Cu") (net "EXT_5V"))
 (segment (start 36.1262 35.6983) (end 36.7279 36.3) (width 0.2) (layer "F.Cu") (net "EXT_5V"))
 (segment (start 44.9161 37.3339) (end 39.9 37.3339) (width 0.2) (layer "F.Cu") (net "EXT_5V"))
 (segment (start 36.7279 36.3) (end 36.9483 36.3) (width 0.2) (layer "F.Cu") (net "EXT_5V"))
 (segment (start 34.75 36.3) (end 34.75 35.6983) (width 0.2) (layer "F.Cu") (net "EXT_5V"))
 (segment (start 33.81 31.27) (end 33.0257 31.27) (width 0.2) (layer "F.Cu") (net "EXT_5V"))
 (segment (start 33.0257 31.2699) (end 31.7843 30.0285) (width 0.2) (layer "F.Cu") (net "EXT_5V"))
 (segment (start 34.75 35.6983) (end 36.1262 35.6983) (width 0.2) (layer "F.Cu") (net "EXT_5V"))
 (segment (start 30.0285 31.7842) (end 33.9426 35.6983) (width 0.2) (layer "F.Cu") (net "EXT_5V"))
 (segment (start 30.0285 30.0285) (end 27.4885 30.0285) (width 0.2) (layer "F.Cu") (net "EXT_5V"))
 (segment (start 34.75 36.9017) (end 35.579 37.7307) (width 0.2) (layer "F.Cu") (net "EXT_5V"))
 (segment (start 30.0285 30.0285) (end 30.0285 31.7842) (width 0.2) (layer "F.Cu") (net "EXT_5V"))
 (segment (start 31.7843 30.0285) (end 30.0285 30.0285) (width 0.2) (layer "F.Cu") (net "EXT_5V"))
 (segment (start 33.9426 35.6983) (end 34.75 35.6983) (width 0.2) (layer "F.Cu") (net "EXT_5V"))
 (segment (start 37.55 33.15) (end 37.55 32.5483) (width 0.2) (layer "F.Cu") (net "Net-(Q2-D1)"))
 (segment (start 33.0063 27.4856) (end 32.8015 27.6904) (width 0.2) (layer "F.Cu") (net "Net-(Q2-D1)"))
 (segment (start 37.05 28.6999) (end 35.8357 27.4856) (width 0.2) (layer "F.Cu") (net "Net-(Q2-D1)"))
 (segment (start 36.9482 32.5483) (end 36.2595 31.8596) (width 0.2) (layer "F.Cu") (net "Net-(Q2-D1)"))
 (segment (start 35.8357 27.4856) (end 33.0063 27.4856) (width 0.2) (layer "F.Cu") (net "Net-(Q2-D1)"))
 (segment (start 37.55 32.5483) (end 36.9482 32.5483) (width 0.2) (layer "F.Cu") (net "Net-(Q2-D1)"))
 (via (at 32.8015 27.6904) (size 0.6) (drill 0.3) (layers "F.Cu" "B.Cu") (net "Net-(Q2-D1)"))
 (via (at 36.2595 31.8596) (size 0.6) (drill 0.3) (layers "F.Cu" "B.Cu") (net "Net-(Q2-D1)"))
 (segment (start 32.8015 27.6904) (end 33.0512 27.4407) (width 0.2) (layer "B.Cu") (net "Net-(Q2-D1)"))
 (segment (start 34.3418 27.4407) (end 36.2595 29.3584) (width 0.2) (layer "B.Cu") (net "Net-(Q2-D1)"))
 (segment (start 36.2595 29.3584) (end 36.2595 31.8596) (width 0.2) (layer "B.Cu") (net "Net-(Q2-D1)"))
 (segment (start 33.0512 27.4407) (end 34.3418 27.4407) (width 0.2) (layer "B.Cu") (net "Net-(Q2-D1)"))
 (segment (start 35.65 36.9017) (end 35.8773 37.129) (width 0.2) (layer "F.Cu") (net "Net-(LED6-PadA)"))
 (segment (start 35.65 36.3) (end 35.65 36.9017) (width 0.2) (layer "F.Cu") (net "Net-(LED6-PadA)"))
 (segment (start 46.4 34.2) (end 47.51 34.2) (width 0.2) (layer "F.Cu") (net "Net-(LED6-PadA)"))
 (segment (start 35.8773 37.129) (end 38.9841 37.129) (width 0.2) (layer "F.Cu") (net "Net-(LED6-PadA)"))
 (via (at 38.9841 37.129) (size 0.6) (drill 0.3) (layers "F.Cu" "B.Cu") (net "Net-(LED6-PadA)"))
 (via (at 47.51 34.2) (size 0.6) (drill 0.3) (layers "F.Cu" "B.Cu") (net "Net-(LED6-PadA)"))
 (segment (start 44.581 37.129) (end 47.51 34.2) (width 0.2) (layer "B.Cu") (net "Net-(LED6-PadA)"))
 (segment (start 38.9841 37.129) (end 44.581 37.129) (width 0.2) (layer "B.Cu") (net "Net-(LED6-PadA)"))
 (segment (start 37.05 31.3001) (end 36.9852 31.2353) (width 0.2) (layer "F.Cu") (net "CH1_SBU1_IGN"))
 (segment (start 33.7536 32.5483) (end 33.5888 32.7131) (width 0.2) (layer "F.Cu") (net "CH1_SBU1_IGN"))
 (segment (start 35.6313 31.6286) (end 35.6313 32.5483) (width 0.2) (layer "F.Cu") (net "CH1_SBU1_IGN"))
 (segment (start 40.35 30) (end 40.35 29.1772) (width 0.2) (layer "F.Cu") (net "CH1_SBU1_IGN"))
 (segment (start 40.35 29.1772) (end 40.3499 29.1772) (width 0.2) (layer "F.Cu") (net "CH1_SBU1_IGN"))
 (segment (start 36.2517 33.15) (end 36.2517 33.0001) (width 0.2) (layer "F.Cu") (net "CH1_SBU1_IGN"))
 (segment (start 36.9852 31.2353) (end 36.0246 31.2353) (width 0.2) (layer "F.Cu") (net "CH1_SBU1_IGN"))
 (segment (start 35.7999 32.5483) (end 35.6313 32.5483) (width 0.2) (layer "F.Cu") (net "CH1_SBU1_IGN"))
 (segment (start 35.65 33.15) (end 36.2517 33.15) (width 0.2) (layer "F.Cu") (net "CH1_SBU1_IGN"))
 (segment (start 36.0246 31.2353) (end 35.6313 31.6286) (width 0.2) (layer "F.Cu") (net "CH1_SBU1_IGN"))
 (segment (start 36.2517 33.0001) (end 35.7999 32.5483) (width 0.2) (layer "F.Cu") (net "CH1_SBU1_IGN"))
 (segment (start 35.6313 32.5483) (end 33.7536 32.5483) (width 0.2) (layer "F.Cu") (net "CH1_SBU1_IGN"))
 (via (at 40.3499 29.1772) (size 0.6) (drill 0.3) (layers "F.Cu" "B.Cu") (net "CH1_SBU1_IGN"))
 (via (at 33.5888 32.7131) (size 0.6) (drill 0.3) (layers "F.Cu" "B.Cu") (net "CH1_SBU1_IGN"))
 (segment (start 33.5888 32.7131) (end 36.814 32.7131) (width 0.2) (layer "B.Cu") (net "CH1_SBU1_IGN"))
 (segment (start 30.1731 32.7131) (end 33.5888 32.7131) (width 0.2) (layer "B.Cu") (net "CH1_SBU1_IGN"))
 (segment (start 28.73 31.27) (end 30.1731 32.7131) (width 0.2) (layer "B.Cu") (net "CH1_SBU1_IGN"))
 (segment (start 36.814 32.7131) (end 40.3499 29.1772) (width 0.2) (layer "B.Cu") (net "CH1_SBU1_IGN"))
 (segment (start 42.65 34.15) (end 41.9483 34.15) (width 0.2) (layer "F.Cu") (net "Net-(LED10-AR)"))
 (segment (start 41.9449 34.1534) (end 41.9483 34.15) (width 0.2) (layer "F.Cu") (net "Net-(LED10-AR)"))
 (segment (start 35.1517 34.1534) (end 41.9449 34.1534) (width 0.2) (layer "F.Cu") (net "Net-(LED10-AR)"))
 (segment (start 34.75 33.15) (end 34.75 33.7517) (width 0.2) (layer "F.Cu") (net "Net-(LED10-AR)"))
 (segment (start 34.75 33.7517) (end 35.1517 34.1534) (width 0.2) (layer "F.Cu") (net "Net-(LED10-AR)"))
 (segment (start 45.3483 29.3982) (end 45.2753 29.3252) (width 0.2) (layer "F.Cu") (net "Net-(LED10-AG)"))
 (segment (start 45.95 30) (end 45.3483 30) (width 0.2) (layer "F.Cu") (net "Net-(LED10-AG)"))
 (segment (start 44.55 33.1737) (end 44.55 34.15) (width 0.2) (layer "F.Cu") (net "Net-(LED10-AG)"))
 (segment (start 45.3483 30) (end 45.3483 29.3982) (width 0.2) (layer "F.Cu") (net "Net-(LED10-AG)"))
 (via (at 45.2753 29.3252) (size 0.6) (drill 0.3) (layers "F.Cu" "B.Cu") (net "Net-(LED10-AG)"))
 (via (at 44.55 33.1737) (size 0.6) (drill 0.3) (layers "F.Cu" "B.Cu") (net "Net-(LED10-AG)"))
 (segment (start 44.55 33.1737) (end 44.55 30.0505) (width 0.2) (layer "B.Cu") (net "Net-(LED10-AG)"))
 (segment (start 44.55 30.0505) (end 45.2753 29.3252) (width 0.2) (layer "B.Cu") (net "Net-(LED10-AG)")))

